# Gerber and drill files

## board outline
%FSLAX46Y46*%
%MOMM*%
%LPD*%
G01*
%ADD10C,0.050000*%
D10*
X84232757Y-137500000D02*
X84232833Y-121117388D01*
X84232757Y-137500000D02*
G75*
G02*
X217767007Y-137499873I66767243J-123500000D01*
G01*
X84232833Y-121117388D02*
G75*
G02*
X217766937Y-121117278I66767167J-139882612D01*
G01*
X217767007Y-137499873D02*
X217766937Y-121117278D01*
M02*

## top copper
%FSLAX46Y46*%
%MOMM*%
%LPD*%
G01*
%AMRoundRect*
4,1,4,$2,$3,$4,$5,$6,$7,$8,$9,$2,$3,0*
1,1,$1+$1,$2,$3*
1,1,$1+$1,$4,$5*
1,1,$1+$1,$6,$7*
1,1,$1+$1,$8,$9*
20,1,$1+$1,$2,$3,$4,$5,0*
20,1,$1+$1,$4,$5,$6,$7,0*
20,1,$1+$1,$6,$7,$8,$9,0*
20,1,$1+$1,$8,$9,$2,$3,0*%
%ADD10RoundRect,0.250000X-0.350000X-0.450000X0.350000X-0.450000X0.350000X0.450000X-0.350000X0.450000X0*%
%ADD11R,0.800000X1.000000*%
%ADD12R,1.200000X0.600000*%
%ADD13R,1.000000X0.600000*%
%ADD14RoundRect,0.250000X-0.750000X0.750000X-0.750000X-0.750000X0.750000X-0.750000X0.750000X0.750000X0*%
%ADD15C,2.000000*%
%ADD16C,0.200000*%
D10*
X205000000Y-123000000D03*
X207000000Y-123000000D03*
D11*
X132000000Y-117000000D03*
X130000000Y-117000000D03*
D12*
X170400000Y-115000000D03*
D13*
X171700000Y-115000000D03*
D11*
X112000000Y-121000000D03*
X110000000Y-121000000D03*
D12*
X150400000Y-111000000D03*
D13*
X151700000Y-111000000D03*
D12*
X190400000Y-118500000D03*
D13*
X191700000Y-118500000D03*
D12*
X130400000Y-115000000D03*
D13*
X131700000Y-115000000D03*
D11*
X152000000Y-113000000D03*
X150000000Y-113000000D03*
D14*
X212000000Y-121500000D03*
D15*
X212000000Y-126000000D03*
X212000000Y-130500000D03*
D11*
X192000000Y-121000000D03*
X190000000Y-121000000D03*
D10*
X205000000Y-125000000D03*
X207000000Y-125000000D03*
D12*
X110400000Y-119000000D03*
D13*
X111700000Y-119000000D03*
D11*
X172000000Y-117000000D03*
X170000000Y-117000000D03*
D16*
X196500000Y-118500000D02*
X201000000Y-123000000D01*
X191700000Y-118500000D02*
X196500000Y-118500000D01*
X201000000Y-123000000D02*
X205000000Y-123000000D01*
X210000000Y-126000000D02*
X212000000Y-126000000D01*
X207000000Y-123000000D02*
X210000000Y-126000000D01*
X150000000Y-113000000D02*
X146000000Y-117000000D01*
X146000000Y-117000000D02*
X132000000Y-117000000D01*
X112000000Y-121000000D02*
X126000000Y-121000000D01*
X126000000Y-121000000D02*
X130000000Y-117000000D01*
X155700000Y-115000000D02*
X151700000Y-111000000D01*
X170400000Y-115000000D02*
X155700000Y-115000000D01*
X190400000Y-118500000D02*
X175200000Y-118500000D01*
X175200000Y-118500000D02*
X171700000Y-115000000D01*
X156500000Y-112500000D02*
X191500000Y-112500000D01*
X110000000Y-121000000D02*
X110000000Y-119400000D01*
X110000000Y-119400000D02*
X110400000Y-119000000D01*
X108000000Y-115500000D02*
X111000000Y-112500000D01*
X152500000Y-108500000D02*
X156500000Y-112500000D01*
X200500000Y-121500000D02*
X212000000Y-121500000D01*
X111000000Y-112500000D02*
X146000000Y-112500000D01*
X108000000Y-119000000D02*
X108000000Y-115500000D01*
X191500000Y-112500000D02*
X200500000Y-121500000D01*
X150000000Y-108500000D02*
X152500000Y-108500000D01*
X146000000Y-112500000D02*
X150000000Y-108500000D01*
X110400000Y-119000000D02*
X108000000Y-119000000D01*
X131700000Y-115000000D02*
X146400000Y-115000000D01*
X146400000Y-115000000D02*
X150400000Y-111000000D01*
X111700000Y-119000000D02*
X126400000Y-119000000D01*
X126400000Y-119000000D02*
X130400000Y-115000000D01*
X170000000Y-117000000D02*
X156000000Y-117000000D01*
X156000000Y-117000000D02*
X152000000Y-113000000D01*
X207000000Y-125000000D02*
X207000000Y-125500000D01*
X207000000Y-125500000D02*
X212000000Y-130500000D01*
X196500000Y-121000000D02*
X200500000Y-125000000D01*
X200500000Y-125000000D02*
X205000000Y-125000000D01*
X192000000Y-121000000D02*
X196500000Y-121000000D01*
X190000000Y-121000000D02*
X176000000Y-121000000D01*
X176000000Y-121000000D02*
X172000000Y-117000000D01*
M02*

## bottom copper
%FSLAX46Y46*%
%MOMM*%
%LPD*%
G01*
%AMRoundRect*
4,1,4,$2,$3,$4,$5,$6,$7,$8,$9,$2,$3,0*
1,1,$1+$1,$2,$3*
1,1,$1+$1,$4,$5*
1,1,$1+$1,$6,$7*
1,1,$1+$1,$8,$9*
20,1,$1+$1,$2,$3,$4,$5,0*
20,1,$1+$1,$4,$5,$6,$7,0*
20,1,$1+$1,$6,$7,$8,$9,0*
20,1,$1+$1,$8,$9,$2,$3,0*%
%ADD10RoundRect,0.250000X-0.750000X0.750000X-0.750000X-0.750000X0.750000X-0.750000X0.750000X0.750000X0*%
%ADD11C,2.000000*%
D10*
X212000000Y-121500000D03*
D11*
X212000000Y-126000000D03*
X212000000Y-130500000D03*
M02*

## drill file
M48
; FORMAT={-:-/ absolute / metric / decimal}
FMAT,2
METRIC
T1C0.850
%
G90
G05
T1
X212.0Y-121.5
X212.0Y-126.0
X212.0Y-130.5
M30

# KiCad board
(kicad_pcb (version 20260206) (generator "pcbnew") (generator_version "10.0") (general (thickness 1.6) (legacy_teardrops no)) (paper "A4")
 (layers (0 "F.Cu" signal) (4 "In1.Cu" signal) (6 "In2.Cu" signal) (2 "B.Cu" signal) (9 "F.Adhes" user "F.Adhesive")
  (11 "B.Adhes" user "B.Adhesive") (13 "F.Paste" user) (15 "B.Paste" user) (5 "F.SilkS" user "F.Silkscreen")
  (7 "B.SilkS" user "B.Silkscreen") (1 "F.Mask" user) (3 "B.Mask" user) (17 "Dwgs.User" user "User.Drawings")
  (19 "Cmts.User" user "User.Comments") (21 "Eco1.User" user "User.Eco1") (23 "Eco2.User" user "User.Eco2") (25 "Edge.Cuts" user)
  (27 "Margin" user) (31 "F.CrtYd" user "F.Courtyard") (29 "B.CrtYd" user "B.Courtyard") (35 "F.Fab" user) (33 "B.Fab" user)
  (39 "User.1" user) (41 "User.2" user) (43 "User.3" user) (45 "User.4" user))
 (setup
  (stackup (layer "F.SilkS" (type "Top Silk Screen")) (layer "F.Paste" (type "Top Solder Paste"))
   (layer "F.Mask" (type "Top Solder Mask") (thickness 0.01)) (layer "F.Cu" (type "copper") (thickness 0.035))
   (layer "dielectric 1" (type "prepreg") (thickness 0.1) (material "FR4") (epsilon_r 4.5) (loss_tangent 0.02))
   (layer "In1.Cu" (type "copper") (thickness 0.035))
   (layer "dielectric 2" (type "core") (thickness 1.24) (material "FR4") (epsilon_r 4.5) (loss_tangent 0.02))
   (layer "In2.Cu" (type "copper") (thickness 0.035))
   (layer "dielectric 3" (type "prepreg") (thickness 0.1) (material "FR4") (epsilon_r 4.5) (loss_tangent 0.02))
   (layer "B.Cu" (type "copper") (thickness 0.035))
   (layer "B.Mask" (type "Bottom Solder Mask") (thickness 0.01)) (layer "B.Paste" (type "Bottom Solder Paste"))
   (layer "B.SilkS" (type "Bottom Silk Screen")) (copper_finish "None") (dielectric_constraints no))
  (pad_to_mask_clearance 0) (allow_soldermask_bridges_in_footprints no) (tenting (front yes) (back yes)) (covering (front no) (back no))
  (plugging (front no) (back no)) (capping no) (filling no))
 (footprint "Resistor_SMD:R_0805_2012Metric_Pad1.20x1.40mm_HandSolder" (layer "F.Cu") (at 206 123)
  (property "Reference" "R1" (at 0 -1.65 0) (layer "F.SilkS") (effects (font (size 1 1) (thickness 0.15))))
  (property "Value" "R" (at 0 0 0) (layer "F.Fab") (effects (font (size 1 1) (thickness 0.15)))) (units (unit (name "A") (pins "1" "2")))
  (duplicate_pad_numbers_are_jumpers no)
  (pad "1" smd roundrect (at -1 0) (size 1.2 1.4) (layers "F.Cu" "F.Mask" "F.Paste") (roundrect_rratio 0.208333) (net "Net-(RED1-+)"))
  (pad "2" smd roundrect (at 1 0) (size 1.2 1.4) (layers "F.Cu" "F.Mask" "F.Paste") (roundrect_rratio 0.208333) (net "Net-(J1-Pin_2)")))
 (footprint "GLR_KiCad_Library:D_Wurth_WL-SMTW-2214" (layer "F.Cu") (at 131 117 180)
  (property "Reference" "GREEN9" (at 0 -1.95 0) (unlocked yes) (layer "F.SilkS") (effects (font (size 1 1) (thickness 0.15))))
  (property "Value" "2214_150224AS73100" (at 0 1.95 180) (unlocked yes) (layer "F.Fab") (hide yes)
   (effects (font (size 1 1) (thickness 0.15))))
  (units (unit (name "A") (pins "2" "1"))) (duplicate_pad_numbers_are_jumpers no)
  (pad "1" smd rect (at -1 0 180) (size 0.8 1) (layers "F.Cu" "F.Mask" "F.Paste") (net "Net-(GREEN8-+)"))
  (pad "2" smd rect (at 1 0 180) (size 0.8 1) (layers "F.Cu" "F.Mask" "F.Paste") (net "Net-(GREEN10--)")))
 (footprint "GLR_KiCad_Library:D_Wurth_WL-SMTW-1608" (layer "F.Cu") (at 171 115)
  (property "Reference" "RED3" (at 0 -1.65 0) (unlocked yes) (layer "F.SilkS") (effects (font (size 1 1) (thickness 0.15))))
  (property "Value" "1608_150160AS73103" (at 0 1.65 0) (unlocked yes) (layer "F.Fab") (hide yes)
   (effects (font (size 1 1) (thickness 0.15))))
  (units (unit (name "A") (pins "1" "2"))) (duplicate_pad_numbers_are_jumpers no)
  (pad "1" smd rect (at -0.6 0) (size 1.2 0.6) (layers "F.Cu" "F.Mask" "F.Paste") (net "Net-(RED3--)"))
  (pad "2" smd rect (at 0.7 0) (size 1 0.6) (layers "F.Cu" "F.Mask" "F.Paste") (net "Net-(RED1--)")))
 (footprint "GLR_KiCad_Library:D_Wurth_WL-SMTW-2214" (layer "F.Cu") (at 111 121 180)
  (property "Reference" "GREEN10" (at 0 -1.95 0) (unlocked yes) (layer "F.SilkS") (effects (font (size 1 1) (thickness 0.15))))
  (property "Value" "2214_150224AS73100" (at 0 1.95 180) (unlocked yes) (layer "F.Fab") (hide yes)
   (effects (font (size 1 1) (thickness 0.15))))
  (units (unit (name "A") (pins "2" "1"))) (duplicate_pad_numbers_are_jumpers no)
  (pad "1" smd rect (at -1 0 180) (size 0.8 1) (layers "F.Cu" "F.Mask" "F.Paste") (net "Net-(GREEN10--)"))
  (pad "2" smd rect (at 1 0 180) (size 0.8 1) (layers "F.Cu" "F.Mask" "F.Paste") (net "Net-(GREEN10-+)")))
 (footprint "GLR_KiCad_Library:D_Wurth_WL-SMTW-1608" (layer "F.Cu") (at 151 111)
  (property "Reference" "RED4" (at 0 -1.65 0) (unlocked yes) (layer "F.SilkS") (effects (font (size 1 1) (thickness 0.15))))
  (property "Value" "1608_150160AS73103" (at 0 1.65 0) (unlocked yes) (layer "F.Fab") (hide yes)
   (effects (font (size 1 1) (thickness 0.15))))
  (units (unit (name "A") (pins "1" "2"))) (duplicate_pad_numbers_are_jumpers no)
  (pad "1" smd rect (at -0.6 0) (size 1.2 0.6) (layers "F.Cu" "F.Mask" "F.Paste") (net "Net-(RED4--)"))
  (pad "2" smd rect (at 0.7 0) (size 1 0.6) (layers "F.Cu" "F.Mask" "F.Paste") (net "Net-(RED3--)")))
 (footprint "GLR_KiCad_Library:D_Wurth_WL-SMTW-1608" (layer "F.Cu") (at 191 118.5)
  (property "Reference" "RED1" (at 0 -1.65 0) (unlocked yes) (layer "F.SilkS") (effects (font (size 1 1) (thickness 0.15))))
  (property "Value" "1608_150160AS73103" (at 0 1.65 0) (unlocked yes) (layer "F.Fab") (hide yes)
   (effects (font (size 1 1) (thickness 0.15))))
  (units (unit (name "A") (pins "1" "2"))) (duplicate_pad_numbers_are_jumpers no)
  (pad "1" smd rect (at -0.6 0) (size 1.2 0.6) (layers "F.Cu" "F.Mask" "F.Paste") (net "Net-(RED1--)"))
  (pad "2" smd rect (at 0.7 0) (size 1 0.6) (layers "F.Cu" "F.Mask" "F.Paste") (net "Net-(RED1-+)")))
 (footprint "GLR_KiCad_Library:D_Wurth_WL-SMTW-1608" (layer "F.Cu") (at 131 115)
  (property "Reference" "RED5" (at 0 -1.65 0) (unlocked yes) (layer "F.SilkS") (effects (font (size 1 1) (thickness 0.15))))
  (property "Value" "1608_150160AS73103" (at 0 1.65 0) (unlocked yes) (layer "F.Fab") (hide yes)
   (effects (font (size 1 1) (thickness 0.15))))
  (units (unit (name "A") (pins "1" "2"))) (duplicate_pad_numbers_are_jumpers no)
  (pad "1" smd rect (at -0.6 0) (size 1.2 0.6) (layers "F.Cu" "F.Mask" "F.Paste") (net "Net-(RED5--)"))
  (pad "2" smd rect (at 0.7 0) (size 1 0.6) (layers "F.Cu" "F.Mask" "F.Paste") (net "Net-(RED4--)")))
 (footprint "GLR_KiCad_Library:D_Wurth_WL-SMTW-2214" (layer "F.Cu") (at 151 113 180)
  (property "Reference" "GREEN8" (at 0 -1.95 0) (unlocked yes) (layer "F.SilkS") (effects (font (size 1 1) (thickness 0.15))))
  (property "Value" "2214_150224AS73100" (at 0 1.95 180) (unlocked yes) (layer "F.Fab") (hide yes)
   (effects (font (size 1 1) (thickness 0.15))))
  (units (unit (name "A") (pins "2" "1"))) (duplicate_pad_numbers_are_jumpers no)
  (pad "1" smd rect (at -1 0 180) (size 0.8 1) (layers "F.Cu" "F.Mask" "F.Paste") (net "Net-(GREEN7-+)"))
  (pad "2" smd rect (at 1 0 180) (size 0.8 1) (layers "F.Cu" "F.Mask" "F.Paste") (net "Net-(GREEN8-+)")))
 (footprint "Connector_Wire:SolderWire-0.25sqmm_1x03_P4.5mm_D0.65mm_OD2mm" (layer "F.Cu") (at 212 121.5 -90)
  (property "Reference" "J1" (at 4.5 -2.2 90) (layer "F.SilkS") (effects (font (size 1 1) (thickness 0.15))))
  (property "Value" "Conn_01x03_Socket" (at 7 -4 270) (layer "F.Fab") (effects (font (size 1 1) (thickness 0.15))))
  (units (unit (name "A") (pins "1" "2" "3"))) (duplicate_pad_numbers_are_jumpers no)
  (pad "1" thru_hole roundrect (at 0 0 270) (size 2 2) (drill 0.85) (layers "*.Cu" "*.Mask") (remove_unused_layers no)
   (roundrect_rratio 0.125) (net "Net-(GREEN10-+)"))
  (pad "2" thru_hole circle (at 4.5 0 270) (size 2 2) (drill 0.85) (layers "*.Cu" "*.Mask") (remove_unused_layers no) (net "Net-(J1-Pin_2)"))
  (pad "3" thru_hole circle (at 9 0 270) (size 2 2) (drill 0.85) (layers "*.Cu" "*.Mask") (remove_unused_layers no) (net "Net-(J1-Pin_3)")))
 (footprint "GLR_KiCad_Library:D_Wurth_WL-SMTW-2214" (layer "F.Cu") (at 191 121 180)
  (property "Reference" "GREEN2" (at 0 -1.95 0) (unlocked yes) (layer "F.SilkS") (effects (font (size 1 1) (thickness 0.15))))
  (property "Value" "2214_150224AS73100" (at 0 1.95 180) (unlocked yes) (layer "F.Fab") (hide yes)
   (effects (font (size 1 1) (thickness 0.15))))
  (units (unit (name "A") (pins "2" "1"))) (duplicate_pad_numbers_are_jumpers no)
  (pad "1" smd rect (at -1 0 180) (size 0.8 1) (layers "F.Cu" "F.Mask" "F.Paste") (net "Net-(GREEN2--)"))
  (pad "2" smd rect (at 1 0 180) (size 0.8 1) (layers "F.Cu" "F.Mask" "F.Paste") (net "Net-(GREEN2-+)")))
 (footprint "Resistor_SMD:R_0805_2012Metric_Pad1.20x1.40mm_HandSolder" (layer "F.Cu") (at 206 125)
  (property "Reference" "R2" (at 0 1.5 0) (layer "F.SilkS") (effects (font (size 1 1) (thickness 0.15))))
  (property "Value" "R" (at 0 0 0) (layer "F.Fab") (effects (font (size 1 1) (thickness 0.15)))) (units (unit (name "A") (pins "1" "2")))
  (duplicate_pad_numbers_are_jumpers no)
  (pad "1" smd roundrect (at -1 0) (size 1.2 1.4) (layers "F.Cu" "F.Mask" "F.Paste") (roundrect_rratio 0.208333) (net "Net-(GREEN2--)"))
  (pad "2" smd roundrect (at 1 0) (size 1.2 1.4) (layers "F.Cu" "F.Mask" "F.Paste") (roundrect_rratio 0.208333) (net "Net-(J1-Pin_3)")))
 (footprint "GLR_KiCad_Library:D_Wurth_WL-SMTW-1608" (layer "F.Cu") (at 111 119)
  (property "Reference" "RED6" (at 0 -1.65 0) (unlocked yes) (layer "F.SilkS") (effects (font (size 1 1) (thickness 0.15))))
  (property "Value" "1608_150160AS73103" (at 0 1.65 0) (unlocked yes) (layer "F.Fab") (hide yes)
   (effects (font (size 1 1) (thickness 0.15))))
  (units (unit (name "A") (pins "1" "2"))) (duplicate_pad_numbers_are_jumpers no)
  (pad "1" smd rect (at -0.6 0) (size 1.2 0.6) (layers "F.Cu" "F.Mask" "F.Paste") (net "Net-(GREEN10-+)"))
  (pad "2" smd rect (at 0.7 0) (size 1 0.6) (layers "F.Cu" "F.Mask" "F.Paste") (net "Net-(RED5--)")))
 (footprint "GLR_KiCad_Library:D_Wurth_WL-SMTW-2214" (layer "F.Cu") (at 171 117 180)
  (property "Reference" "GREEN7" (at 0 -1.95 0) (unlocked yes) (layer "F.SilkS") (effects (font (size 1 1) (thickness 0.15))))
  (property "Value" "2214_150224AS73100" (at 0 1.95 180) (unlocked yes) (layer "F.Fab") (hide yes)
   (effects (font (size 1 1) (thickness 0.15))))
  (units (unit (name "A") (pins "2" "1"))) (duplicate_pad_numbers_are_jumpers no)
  (pad "1" smd rect (at -1 0 180) (size 0.8 1) (layers "F.Cu" "F.Mask" "F.Paste") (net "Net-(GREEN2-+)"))
  (pad "2" smd rect (at 1 0 180) (size 0.8 1) (layers "F.Cu" "F.Mask" "F.Paste") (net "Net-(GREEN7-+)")))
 (gr_line (start 84.232757 137.5) (end 84.232833 121.117388) (stroke (width 0.05) (type default)) (locked yes) (layer "Edge.Cuts"))
 (gr_arc (start 84.232757 137.5) (mid 150.999866 120.607284) (end 217.767007 137.499873) (stroke (width 0.05) (type default)) (locked yes)
  (layer "Edge.Cuts"))
 (gr_arc (start 84.232833 121.117388) (mid 150.999873 106.000001) (end 217.766937 121.117278) (stroke (width 0.05) (type default))
  (locked yes) (layer "Edge.Cuts"))
 (gr_line (start 217.767007 137.499873) (end 217.766937 121.117278) (stroke (width 0.05) (type default)) (locked yes) (layer "Edge.Cuts"))
 (segment (start 196.5 118.5) (end 201 123) (width 0.2) (layer "F.Cu") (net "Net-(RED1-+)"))
 (segment (start 191.7 118.5) (end 196.5 118.5) (width 0.2) (layer "F.Cu") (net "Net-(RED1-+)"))
 (segment (start 201 123) (end 205 123) (width 0.2) (layer "F.Cu") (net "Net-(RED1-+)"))
 (segment (start 210 126) (end 212 126) (width 0.2) (layer "F.Cu") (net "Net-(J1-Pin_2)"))
 (segment (start 207 123) (end 210 126) (width 0.2) (layer "F.Cu") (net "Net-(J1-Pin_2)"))
 (segment (start 150 113) (end 146 117) (width 0.2) (layer "F.Cu") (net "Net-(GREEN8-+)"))
 (segment (start 146 117) (end 132 117) (width 0.2) (layer "F.Cu") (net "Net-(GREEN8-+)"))
 (segment (start 112 121) (end 126 121) (width 0.2) (layer "F.Cu") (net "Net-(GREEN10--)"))
 (segment (start 126 121) (end 130 117) (width 0.2) (layer "F.Cu") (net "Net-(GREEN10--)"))
 (segment (start 155.7 115) (end 151.7 111) (width 0.2) (layer "F.Cu") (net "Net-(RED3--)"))
 (segment (start 170.4 115) (end 155.7 115) (width 0.2) (layer "F.Cu") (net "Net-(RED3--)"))
 (segment (start 190.4 118.5) (end 175.2 118.5) (width 0.2) (layer "F.Cu") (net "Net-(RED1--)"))
 (segment (start 175.2 118.5) (end 171.7 115) (width 0.2) (layer "F.Cu") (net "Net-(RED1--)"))
 (segment (start 156.5 112.5) (end 191.5 112.5) (width 0.2) (layer "F.Cu") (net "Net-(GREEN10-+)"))
 (segment (start 110 121) (end 110 119.4) (width 0.2) (layer "F.Cu") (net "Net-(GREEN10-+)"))
 (segment (start 110 119.4) (end 110.4 119) (width 0.2) (layer "F.Cu") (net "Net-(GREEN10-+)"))
 (segment (start 108 115.5) (end 111 112.5) (width 0.2) (layer "F.Cu") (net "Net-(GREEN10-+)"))
 (segment (start 152.5 108.5) (end 156.5 112.5) (width 0.2) (layer "F.Cu") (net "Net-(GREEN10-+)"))
 (segment (start 200.5 121.5) (end 212 121.5) (width 0.2) (layer "F.Cu") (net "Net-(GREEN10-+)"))
 (segment (start 111 112.5) (end 146 112.5) (width 0.2) (layer "F.Cu") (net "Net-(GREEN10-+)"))
 (segment (start 108 119) (end 108 115.5) (width 0.2) (layer "F.Cu") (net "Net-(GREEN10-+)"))
 (segment (start 191.5 112.5) (end 200.5 121.5) (width 0.2) (layer "F.Cu") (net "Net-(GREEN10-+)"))
 (segment (start 150 108.5) (end 152.5 108.5) (width 0.2) (layer "F.Cu") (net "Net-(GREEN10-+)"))
 (segment (start 146 112.5) (end 150 108.5) (width 0.2) (layer "F.Cu") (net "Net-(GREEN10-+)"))
 (segment (start 110.4 119) (end 108 119) (width 0.2) (layer "F.Cu") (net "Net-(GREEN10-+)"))
 (segment (start 131.7 115) (end 146.4 115) (width 0.2) (layer "F.Cu") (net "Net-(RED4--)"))
 (segment (start 146.4 115) (end 150.4 111) (width 0.2) (layer "F.Cu") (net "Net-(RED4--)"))
 (segment (start 111.7 119) (end 126.4 119) (width 0.2) (layer "F.Cu") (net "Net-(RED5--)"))
 (segment (start 126.4 119) (end 130.4 115) (width 0.2) (layer "F.Cu") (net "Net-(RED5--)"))
 (segment (start 170 117) (end 156 117) (width 0.2) (layer "F.Cu") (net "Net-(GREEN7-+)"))
 (segment (start 156 117) (end 152 113) (width 0.2) (layer "F.Cu") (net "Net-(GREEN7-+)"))
 (segment (start 207 125) (end 207 125.5) (width 0.2) (layer "F.Cu") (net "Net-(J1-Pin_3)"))
 (segment (start 207 125.5) (end 212 130.5) (width 0.2) (layer "F.Cu") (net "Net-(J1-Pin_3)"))
 (segment (start 196.5 121) (end 200.5 125) (width 0.2) (layer "F.Cu") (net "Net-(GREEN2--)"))
 (segment (start 200.5 125) (end 205 125) (width 0.2) (layer "F.Cu") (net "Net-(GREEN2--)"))
 (segment (start 192 121) (end 196.5 121) (width 0.2) (layer "F.Cu") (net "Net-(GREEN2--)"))
 (segment (start 190 121) (end 176 121) (width 0.2) (layer "F.Cu") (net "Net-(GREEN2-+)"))
 (segment (start 176 121) (end 172 117) (width 0.2) (layer "F.Cu") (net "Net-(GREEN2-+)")))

